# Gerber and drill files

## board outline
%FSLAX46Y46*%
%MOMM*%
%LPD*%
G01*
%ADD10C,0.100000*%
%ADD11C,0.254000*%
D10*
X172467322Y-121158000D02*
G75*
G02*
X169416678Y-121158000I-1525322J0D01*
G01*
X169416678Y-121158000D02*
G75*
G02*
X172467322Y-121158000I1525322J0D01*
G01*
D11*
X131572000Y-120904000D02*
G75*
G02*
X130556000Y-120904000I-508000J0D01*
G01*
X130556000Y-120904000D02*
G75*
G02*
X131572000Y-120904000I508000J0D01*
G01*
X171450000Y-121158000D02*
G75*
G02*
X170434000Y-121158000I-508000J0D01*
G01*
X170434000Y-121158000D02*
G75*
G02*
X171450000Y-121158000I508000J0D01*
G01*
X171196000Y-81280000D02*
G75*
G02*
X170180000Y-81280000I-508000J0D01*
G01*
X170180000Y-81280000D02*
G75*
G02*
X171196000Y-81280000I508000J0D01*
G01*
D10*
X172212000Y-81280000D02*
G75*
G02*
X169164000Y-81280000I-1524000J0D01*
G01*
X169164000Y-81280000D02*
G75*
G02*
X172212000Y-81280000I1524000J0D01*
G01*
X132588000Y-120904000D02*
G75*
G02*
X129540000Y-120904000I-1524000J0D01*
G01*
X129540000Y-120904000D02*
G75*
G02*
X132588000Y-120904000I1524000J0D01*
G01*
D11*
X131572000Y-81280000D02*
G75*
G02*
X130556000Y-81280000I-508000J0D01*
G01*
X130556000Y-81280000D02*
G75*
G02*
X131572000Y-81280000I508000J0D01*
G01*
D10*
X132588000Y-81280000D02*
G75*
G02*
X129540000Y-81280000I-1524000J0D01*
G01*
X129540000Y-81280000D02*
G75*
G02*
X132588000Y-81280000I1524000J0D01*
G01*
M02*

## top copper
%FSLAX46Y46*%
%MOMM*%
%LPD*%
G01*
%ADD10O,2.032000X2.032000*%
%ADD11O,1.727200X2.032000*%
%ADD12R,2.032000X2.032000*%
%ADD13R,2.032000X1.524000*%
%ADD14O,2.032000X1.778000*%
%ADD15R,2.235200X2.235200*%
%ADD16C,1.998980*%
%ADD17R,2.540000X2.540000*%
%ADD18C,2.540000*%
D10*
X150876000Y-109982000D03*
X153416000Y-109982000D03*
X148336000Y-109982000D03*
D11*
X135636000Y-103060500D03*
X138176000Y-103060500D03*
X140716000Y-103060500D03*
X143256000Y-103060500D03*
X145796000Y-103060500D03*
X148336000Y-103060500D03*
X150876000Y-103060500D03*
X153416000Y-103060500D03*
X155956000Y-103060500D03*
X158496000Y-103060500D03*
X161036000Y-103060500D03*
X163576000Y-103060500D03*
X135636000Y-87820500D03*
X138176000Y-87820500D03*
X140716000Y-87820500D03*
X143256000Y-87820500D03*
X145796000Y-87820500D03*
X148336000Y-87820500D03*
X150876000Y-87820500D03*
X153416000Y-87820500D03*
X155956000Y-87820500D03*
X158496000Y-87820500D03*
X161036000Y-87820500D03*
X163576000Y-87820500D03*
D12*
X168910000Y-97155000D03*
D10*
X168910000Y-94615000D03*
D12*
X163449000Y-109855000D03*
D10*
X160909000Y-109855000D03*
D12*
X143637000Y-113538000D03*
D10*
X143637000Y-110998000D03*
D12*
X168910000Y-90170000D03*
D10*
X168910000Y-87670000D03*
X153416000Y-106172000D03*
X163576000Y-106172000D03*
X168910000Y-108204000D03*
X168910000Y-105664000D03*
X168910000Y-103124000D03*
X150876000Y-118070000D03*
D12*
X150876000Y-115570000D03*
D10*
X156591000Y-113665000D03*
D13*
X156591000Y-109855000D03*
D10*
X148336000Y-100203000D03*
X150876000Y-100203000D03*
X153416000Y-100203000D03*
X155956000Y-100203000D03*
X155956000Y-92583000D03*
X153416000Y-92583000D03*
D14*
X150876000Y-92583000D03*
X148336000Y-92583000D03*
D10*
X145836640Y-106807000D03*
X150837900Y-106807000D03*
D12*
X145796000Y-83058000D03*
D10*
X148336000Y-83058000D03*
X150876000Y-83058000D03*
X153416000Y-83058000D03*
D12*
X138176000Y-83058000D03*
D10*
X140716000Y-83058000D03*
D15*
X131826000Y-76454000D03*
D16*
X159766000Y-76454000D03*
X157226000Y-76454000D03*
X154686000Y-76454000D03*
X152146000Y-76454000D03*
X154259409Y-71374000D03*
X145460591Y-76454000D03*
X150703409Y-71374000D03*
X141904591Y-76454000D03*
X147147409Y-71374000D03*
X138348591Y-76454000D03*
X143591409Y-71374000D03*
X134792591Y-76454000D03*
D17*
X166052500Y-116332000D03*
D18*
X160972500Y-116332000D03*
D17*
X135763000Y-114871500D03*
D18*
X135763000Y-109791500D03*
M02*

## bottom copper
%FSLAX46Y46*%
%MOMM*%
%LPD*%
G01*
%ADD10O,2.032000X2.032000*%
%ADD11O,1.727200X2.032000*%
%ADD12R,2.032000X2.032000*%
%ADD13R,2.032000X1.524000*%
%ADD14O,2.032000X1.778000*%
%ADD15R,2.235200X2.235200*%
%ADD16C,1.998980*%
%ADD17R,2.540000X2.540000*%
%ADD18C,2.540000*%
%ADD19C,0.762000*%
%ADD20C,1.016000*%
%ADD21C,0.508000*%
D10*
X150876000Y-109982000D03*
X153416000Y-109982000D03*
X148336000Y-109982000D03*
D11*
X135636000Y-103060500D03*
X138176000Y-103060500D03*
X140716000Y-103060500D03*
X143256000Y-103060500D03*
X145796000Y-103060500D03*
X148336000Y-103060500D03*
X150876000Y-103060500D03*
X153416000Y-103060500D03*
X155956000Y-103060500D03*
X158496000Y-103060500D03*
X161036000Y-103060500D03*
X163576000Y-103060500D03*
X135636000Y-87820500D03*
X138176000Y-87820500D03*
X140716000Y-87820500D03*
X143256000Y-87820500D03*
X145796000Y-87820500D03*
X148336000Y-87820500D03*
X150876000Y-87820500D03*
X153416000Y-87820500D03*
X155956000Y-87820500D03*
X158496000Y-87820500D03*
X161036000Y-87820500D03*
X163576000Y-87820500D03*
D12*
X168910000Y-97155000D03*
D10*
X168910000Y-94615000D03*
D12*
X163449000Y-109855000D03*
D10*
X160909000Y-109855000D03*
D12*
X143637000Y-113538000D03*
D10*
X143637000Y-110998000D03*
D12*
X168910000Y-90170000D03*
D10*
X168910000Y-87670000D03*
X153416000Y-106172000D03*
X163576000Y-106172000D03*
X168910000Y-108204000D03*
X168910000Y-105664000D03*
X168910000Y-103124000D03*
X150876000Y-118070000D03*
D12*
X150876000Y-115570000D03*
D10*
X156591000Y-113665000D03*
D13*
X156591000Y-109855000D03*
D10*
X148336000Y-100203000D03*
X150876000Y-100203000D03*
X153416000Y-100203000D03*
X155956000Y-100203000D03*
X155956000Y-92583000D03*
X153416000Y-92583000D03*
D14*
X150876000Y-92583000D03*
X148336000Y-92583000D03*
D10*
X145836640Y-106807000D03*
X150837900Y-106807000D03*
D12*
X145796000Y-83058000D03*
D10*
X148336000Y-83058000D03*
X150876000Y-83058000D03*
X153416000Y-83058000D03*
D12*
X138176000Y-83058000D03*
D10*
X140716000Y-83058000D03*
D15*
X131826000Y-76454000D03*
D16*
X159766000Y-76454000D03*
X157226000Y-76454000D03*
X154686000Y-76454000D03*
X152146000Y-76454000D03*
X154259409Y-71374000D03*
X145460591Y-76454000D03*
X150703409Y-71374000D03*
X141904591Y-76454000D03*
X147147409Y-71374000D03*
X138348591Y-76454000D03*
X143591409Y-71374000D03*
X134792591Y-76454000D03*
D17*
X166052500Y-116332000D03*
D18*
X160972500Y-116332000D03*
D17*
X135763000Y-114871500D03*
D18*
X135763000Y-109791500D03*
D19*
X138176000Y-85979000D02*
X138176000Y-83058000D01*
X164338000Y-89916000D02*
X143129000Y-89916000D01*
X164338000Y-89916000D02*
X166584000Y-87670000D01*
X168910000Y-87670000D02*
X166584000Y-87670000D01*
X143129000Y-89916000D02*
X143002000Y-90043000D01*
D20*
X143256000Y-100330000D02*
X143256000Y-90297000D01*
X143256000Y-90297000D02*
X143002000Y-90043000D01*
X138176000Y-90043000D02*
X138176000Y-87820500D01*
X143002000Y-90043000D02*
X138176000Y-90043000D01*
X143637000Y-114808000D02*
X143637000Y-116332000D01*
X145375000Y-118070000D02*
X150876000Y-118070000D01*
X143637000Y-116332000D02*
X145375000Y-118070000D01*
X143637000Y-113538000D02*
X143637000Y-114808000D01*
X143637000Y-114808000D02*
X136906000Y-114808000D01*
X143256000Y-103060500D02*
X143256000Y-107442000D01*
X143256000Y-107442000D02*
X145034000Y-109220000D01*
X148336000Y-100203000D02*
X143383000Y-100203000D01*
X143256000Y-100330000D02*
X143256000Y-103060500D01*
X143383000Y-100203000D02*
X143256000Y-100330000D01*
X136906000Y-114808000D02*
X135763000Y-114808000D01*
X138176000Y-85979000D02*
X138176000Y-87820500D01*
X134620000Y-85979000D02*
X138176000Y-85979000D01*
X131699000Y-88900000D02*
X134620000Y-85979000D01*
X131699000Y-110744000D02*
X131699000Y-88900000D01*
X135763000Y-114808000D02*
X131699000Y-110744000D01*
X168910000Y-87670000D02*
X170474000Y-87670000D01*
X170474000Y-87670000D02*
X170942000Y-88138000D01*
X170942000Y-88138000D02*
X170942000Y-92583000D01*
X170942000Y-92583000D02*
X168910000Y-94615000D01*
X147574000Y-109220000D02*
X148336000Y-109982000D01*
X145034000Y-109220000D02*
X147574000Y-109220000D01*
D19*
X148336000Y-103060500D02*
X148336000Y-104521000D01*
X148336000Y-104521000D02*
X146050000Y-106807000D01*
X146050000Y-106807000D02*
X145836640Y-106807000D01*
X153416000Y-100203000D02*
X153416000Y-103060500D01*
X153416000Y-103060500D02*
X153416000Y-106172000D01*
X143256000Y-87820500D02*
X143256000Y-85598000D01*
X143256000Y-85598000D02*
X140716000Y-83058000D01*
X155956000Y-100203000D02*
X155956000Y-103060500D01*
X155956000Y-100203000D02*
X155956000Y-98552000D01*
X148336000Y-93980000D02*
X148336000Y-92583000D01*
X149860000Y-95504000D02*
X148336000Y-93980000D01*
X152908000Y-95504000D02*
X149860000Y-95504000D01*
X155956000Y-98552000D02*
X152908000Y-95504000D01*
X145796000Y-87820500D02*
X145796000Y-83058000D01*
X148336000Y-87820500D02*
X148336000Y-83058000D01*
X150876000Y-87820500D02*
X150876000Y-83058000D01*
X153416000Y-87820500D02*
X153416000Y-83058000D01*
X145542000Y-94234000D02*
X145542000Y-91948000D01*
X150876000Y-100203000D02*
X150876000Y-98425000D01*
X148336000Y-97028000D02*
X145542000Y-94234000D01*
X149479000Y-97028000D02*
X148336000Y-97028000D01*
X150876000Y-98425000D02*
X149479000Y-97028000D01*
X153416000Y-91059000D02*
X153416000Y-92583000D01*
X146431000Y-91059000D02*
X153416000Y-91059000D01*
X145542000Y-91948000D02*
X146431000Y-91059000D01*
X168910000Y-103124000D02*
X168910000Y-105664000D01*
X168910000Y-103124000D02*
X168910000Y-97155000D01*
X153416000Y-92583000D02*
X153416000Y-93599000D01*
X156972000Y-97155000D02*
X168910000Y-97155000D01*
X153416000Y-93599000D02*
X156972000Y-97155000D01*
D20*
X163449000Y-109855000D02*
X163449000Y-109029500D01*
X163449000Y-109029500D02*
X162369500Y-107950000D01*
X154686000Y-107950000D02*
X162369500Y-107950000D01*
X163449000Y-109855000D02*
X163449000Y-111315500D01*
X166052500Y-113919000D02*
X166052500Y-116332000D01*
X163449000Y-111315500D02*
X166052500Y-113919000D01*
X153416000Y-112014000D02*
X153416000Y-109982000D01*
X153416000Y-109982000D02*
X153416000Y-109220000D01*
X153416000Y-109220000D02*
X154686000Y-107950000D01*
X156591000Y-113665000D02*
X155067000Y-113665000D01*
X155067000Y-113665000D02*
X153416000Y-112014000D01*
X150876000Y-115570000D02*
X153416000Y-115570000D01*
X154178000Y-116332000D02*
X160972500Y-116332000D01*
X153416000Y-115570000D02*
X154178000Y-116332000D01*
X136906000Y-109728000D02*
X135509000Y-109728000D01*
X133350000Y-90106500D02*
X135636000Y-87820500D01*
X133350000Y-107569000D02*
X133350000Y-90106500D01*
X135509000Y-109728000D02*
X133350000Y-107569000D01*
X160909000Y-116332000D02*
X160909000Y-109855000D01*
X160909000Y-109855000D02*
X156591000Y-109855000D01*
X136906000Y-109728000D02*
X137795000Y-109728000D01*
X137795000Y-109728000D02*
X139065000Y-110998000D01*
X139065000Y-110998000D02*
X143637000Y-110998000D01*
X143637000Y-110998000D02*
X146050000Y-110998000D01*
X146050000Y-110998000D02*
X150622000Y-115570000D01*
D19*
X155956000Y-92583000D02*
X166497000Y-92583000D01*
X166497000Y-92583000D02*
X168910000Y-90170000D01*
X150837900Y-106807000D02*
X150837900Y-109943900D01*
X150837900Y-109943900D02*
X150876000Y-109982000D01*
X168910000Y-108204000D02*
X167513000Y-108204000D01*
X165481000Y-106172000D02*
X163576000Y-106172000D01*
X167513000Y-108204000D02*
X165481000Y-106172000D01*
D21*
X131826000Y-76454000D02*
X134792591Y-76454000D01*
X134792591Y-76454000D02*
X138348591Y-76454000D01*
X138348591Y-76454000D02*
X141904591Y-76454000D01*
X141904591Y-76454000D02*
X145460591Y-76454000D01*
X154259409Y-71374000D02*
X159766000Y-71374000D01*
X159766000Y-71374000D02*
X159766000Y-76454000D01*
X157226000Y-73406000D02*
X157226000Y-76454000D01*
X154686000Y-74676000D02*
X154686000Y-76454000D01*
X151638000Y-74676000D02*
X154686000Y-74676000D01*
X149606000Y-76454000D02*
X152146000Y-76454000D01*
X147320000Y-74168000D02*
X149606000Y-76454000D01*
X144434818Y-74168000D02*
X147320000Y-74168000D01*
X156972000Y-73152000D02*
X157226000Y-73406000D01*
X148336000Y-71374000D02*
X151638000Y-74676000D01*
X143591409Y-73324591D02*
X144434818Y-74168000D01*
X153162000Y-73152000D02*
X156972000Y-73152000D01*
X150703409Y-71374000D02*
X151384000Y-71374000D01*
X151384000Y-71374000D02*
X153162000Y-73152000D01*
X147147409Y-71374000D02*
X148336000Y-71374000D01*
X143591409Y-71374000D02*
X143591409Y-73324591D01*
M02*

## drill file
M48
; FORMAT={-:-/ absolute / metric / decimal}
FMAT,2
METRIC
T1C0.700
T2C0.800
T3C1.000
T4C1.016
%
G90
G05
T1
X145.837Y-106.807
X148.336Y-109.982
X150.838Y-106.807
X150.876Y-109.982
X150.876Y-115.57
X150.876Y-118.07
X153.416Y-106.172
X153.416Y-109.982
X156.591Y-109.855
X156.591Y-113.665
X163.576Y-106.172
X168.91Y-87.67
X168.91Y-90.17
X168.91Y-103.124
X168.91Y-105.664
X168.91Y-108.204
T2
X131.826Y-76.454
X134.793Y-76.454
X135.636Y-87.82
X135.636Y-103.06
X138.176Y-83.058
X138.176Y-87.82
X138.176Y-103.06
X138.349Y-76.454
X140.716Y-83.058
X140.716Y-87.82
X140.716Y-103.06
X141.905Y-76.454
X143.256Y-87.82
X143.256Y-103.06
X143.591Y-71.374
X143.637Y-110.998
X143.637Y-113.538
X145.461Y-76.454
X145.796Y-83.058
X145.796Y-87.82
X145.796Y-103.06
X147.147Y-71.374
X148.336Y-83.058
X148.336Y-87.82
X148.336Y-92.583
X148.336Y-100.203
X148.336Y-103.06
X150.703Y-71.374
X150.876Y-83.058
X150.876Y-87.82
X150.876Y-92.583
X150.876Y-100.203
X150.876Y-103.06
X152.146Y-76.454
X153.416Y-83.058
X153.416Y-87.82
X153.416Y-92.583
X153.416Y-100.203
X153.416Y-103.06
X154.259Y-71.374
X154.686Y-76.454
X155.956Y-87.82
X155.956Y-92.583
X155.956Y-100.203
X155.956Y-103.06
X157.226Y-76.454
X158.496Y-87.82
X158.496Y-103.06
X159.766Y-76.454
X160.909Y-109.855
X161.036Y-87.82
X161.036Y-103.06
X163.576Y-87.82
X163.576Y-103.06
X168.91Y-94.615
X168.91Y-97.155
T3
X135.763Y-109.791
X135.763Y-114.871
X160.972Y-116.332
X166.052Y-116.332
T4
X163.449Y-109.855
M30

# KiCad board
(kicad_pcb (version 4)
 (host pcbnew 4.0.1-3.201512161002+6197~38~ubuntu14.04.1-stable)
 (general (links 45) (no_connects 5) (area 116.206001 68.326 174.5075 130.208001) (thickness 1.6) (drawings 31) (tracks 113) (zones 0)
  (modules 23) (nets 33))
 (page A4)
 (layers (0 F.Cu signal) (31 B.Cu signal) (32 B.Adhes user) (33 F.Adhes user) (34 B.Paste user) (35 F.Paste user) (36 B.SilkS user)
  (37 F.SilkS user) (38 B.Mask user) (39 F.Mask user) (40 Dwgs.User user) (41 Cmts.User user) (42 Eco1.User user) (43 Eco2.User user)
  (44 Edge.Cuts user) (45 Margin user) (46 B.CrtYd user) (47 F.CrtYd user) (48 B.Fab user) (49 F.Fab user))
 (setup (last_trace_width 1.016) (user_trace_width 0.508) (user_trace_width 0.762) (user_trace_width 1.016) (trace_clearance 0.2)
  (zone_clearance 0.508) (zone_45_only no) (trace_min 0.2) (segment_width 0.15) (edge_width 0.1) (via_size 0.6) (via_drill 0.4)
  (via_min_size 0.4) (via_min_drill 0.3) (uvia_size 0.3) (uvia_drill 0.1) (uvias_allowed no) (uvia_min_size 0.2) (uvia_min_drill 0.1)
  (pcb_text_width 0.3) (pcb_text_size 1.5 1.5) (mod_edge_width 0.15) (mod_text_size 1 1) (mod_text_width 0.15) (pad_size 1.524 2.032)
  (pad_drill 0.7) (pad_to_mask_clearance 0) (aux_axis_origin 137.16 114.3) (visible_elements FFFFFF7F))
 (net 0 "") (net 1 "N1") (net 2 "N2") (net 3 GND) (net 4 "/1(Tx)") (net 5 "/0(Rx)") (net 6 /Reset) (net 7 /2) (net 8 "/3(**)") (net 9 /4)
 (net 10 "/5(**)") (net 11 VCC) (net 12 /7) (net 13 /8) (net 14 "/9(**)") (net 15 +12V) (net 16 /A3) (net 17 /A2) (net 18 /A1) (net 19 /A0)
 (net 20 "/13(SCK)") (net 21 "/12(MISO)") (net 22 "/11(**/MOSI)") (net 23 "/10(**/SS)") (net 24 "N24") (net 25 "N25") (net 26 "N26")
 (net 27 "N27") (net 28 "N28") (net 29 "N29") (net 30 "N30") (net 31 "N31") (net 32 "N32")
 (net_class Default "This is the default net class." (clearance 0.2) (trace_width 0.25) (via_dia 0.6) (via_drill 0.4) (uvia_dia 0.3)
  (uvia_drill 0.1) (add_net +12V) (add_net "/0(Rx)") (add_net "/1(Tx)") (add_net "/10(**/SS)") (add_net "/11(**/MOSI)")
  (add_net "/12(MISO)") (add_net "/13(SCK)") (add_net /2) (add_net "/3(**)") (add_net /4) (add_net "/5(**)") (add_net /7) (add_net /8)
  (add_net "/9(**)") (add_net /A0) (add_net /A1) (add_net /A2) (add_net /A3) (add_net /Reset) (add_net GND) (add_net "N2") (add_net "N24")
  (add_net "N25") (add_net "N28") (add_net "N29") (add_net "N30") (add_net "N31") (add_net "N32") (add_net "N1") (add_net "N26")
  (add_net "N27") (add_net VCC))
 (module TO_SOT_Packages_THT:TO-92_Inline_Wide (layer F.Cu) (at 148.336 109.982)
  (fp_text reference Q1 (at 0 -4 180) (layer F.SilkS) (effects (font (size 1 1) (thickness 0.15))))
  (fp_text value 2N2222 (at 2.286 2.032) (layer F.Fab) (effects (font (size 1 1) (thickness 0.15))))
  (pad 2 thru_hole oval (at 2.54 0) (size 2.032 2.032) (drill 0.7) (layers *.Cu *.Mask F.SilkS) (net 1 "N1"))
  (pad 3 thru_hole oval (at 5.08 0) (size 2.032 2.032) (drill 0.7) (layers *.Cu *.Mask F.SilkS) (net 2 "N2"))
  (pad 1 thru_hole oval (at 0 0) (size 2.032 2.032) (drill 0.7) (layers *.Cu *.Mask F.SilkS) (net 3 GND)))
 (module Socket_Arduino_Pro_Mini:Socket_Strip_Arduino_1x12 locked (layer F.Cu) (at 135.636 103.0605)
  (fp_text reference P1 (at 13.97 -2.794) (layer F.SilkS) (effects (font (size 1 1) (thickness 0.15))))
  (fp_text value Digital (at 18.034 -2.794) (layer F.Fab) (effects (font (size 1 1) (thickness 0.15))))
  (pad 1 thru_hole oval (at 0 0) (size 1.7272 2.032) (drill 0.8) (layers *.Cu *.Mask F.SilkS) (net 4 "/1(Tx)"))
  (pad 2 thru_hole oval (at 2.54 0) (size 1.7272 2.032) (drill 0.8) (layers *.Cu *.Mask F.SilkS) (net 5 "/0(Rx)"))
  (pad 3 thru_hole oval (at 5.08 0) (size 1.7272 2.032) (drill 0.8) (layers *.Cu *.Mask F.SilkS) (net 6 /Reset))
  (pad 4 thru_hole oval (at 7.62 0) (size 1.7272 2.032) (drill 0.8) (layers *.Cu *.Mask F.SilkS) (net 3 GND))
  (pad 5 thru_hole oval (at 10.16 0) (size 1.7272 2.032) (drill 0.8) (layers *.Cu *.Mask F.SilkS) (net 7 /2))
  (pad 6 thru_hole oval (at 12.7 0) (size 1.7272 2.032) (drill 0.8) (layers *.Cu *.Mask F.SilkS) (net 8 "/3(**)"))
  (pad 7 thru_hole oval (at 15.24 0) (size 1.7272 2.032) (drill 0.8) (layers *.Cu *.Mask F.SilkS) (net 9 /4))
  (pad 8 thru_hole oval (at 17.78 0) (size 1.7272 2.032) (drill 0.8) (layers *.Cu *.Mask F.SilkS) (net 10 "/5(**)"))
  (pad 9 thru_hole oval (at 20.32 0) (size 1.7272 2.032) (drill 0.8) (layers *.Cu *.Mask F.SilkS) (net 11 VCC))
  (pad 10 thru_hole oval (at 22.86 0) (size 1.7272 2.032) (drill 0.8) (layers *.Cu *.Mask F.SilkS) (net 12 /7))
  (pad 11 thru_hole oval (at 25.4 0) (size 1.7272 2.032) (drill 0.8) (layers *.Cu *.Mask F.SilkS) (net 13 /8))
  (pad 12 thru_hole oval (at 27.94 0) (size 1.7272 2.032) (drill 0.8) (layers *.Cu *.Mask F.SilkS) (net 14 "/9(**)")))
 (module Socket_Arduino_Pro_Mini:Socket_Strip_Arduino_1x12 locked (layer F.Cu) (at 135.636 87.8205)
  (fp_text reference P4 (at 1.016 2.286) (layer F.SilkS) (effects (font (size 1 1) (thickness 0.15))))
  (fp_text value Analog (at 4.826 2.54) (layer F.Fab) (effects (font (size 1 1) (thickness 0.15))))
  (pad 1 thru_hole oval (at 0 0) (size 1.7272 2.032) (drill 0.8) (layers *.Cu *.Mask F.SilkS) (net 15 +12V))
  (pad 2 thru_hole oval (at 2.54 0) (size 1.7272 2.032) (drill 0.8) (layers *.Cu *.Mask F.SilkS) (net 3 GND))
  (pad 3 thru_hole oval (at 5.08 0) (size 1.7272 2.032) (drill 0.8) (layers *.Cu *.Mask F.SilkS) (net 6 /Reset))
  (pad 4 thru_hole oval (at 7.62 0) (size 1.7272 2.032) (drill 0.8) (layers *.Cu *.Mask F.SilkS) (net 11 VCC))
  (pad 5 thru_hole oval (at 10.16 0) (size 1.7272 2.032) (drill 0.8) (layers *.Cu *.Mask F.SilkS) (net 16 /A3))
  (pad 6 thru_hole oval (at 12.7 0) (size 1.7272 2.032) (drill 0.8) (layers *.Cu *.Mask F.SilkS) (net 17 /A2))
  (pad 7 thru_hole oval (at 15.24 0) (size 1.7272 2.032) (drill 0.8) (layers *.Cu *.Mask F.SilkS) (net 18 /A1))
  (pad 8 thru_hole oval (at 17.78 0) (size 1.7272 2.032) (drill 0.8) (layers *.Cu *.Mask F.SilkS) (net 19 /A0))
  (pad 9 thru_hole oval (at 20.32 0) (size 1.7272 2.032) (drill 0.8) (layers *.Cu *.Mask F.SilkS) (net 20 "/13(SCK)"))
  (pad 10 thru_hole oval (at 22.86 0) (size 1.7272 2.032) (drill 0.8) (layers *.Cu *.Mask F.SilkS) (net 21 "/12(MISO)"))
  (pad 11 thru_hole oval (at 25.4 0) (size 1.7272 2.032) (drill 0.8) (layers *.Cu *.Mask F.SilkS) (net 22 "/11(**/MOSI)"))
  (pad 12 thru_hole oval (at 27.94 0) (size 1.7272 2.032) (drill 0.8) (layers *.Cu *.Mask F.SilkS) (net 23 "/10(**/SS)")))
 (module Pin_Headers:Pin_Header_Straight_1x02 (layer F.Cu) (at 168.91 97.155 180)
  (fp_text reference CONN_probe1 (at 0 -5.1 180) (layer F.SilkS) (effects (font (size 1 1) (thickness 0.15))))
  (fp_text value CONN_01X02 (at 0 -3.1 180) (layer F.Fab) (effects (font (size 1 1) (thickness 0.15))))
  (pad 1 thru_hole rect (at 0 0 180) (size 2.032 2.032) (drill 0.8) (layers *.Cu *.Mask F.SilkS) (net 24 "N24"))
  (pad 2 thru_hole oval (at 0 2.54 180) (size 2.032 2.032) (drill 0.8) (layers *.Cu *.Mask F.SilkS) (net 3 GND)))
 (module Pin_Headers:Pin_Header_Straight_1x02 (layer F.Cu) (at 163.449 109.855 270)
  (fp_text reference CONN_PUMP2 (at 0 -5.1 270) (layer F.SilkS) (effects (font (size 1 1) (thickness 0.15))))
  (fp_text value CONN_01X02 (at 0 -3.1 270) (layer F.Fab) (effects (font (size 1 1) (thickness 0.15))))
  (pad 1 thru_hole rect (at 0 0 270) (size 2.032 2.032) (drill 1.016) (layers *.Cu *.Mask F.SilkS) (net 2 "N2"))
  (pad 2 thru_hole oval (at 0 2.54 270) (size 2.032 2.032) (drill 0.8) (layers *.Cu *.Mask F.SilkS) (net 15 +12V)))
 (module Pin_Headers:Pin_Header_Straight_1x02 (layer F.Cu) (at 143.637 113.538 180)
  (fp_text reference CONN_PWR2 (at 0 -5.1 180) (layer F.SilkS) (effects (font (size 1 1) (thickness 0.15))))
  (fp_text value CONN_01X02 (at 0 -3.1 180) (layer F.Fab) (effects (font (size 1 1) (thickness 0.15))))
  (pad 1 thru_hole rect (at 0 0 180) (size 2.032 2.032) (drill 0.8) (layers *.Cu *.Mask F.SilkS) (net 3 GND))
  (pad 2 thru_hole oval (at 0 2.54 180) (size 2.032 2.032) (drill 0.8) (layers *.Cu *.Mask F.SilkS) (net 15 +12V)))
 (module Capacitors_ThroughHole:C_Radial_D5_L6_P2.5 (layer F.Cu) (at 168.91 90.17 90)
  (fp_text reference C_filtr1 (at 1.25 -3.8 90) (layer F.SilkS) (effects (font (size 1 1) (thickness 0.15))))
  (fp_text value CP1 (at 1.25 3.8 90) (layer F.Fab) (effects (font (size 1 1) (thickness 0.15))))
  (pad 1 thru_hole rect (at 0 0 90) (size 2.032 2.032) (drill 0.7) (layers *.Cu *.Mask F.SilkS) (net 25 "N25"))
  (pad 2 thru_hole oval (at 2.5 0 90) (size 2.032 2.032) (drill 0.7) (layers *.Cu *.Mask F.SilkS) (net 3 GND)))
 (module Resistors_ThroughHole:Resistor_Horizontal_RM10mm (layer F.Cu) (at 158.496 106.172)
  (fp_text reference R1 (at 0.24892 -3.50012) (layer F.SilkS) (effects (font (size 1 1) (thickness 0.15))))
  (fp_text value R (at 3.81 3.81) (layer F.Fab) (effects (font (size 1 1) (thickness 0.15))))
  (pad 1 thru_hole oval (at -5.08 0) (size 2.032 2.032) (drill 0.7) (layers *.Cu *.Mask F.SilkS) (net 10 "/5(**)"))
  (pad 2 thru_hole oval (at 5.08 0) (size 2.032 2.032) (drill 0.7) (layers *.Cu *.Mask F.SilkS) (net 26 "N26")))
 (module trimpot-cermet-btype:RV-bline (layer F.Cu) (at 168.91 105.664 90)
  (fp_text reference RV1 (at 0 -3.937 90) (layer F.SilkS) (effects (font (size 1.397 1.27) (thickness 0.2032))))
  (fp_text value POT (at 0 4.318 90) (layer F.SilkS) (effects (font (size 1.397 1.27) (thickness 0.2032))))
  (pad 1 thru_hole oval (at -2.54 0 90) (size 2.032 2.032) (drill 0.7) (layers *.Cu *.Mask F.SilkS) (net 26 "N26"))
  (pad 2 thru_hole oval (at 0 0 90) (size 2.032 2.032) (drill 0.7) (layers *.Cu *.Mask F.SilkS) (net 24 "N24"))
  (pad 3 thru_hole oval (at 2.54 0 90) (size 2.032 2.032) (drill 0.7) (layers *.Cu *.Mask F.SilkS) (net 24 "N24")))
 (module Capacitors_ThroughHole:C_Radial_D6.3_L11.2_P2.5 (layer F.Cu) (at 150.876 115.57 270)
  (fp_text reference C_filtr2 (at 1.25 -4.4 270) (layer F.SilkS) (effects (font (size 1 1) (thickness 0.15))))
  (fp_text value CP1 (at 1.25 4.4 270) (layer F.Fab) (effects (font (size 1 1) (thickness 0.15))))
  (pad 2 thru_hole oval (at 2.5 0 270) (size 2.032 2.032) (drill 0.7) (layers *.Cu *.Mask F.SilkS) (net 3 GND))
  (pad 1 thru_hole rect (at 0 0 270) (size 2.032 2.032) (drill 0.7) (layers *.Cu *.Mask F.SilkS) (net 15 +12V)))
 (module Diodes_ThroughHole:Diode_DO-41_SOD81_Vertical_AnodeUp (layer F.Cu) (at 156.591 109.855 270)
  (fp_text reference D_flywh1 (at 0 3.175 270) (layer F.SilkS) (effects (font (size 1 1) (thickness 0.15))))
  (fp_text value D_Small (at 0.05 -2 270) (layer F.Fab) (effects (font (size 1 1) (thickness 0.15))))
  (pad 2 thru_hole oval (at 3.81 0 270) (size 2.032 2.032) (drill 0.7) (layers *.Cu *.Mask F.SilkS) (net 2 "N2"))
  (pad 1 thru_hole rect (at 0 0 270) (size 1.524 2.032) (drill 0.7) (layers *.Cu *.Mask F.SilkS) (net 15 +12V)))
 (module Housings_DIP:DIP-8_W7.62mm (layer F.Cu) (at 148.336 100.203 90)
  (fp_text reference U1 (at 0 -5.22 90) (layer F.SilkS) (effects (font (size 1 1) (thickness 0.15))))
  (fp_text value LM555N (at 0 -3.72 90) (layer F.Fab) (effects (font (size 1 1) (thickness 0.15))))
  (pad 1 thru_hole oval (at 0 0 90) (size 2.032 2.032) (drill 0.8) (layers *.Cu *.Mask F.SilkS) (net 3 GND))
  (pad 2 thru_hole oval (at 0 2.54 90) (size 2.032 2.032) (drill 0.8) (layers *.Cu *.Mask F.SilkS) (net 24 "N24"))
  (pad 3 thru_hole oval (at 0 5.08 90) (size 2.032 2.032) (drill 0.8) (layers *.Cu *.Mask F.SilkS) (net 10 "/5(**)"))
  (pad 4 thru_hole oval (at 0 7.62 90) (size 2.032 2.032) (drill 0.8) (layers *.Cu *.Mask F.SilkS) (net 11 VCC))
  (pad 5 thru_hole oval (at 7.62 7.62 90) (size 2.032 2.032) (drill 0.8) (layers *.Cu *.Mask F.SilkS) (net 25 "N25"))
  (pad 6 thru_hole oval (at 7.62 5.08 90) (size 2.032 2.032) (drill 0.8) (layers *.Cu *.Mask F.SilkS) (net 24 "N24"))
  (pad 7 thru_hole oval (at 7.62 2.54 90) (size 1.778 2.032) (drill 0.8) (layers *.Cu *.Mask F.SilkS) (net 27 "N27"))
  (pad 8 thru_hole oval (at 7.62 0 90) (size 1.778 2.032) (drill 0.8) (layers *.Cu *.Mask F.SilkS) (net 11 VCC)))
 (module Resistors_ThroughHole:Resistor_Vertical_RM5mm (layer F.Cu) (at 148.336 106.807)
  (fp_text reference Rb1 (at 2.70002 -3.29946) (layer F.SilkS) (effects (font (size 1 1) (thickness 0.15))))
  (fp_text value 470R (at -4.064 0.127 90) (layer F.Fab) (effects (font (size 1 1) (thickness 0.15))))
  (pad 1 thru_hole oval (at -2.49936 0) (size 2.032 2.032) (drill 0.7) (layers *.Cu *.Mask F.SilkS) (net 8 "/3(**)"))
  (pad 2 thru_hole oval (at 2.5019 0) (size 2.032 2.032) (drill 0.7) (layers *.Cu *.Mask F.SilkS) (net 1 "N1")))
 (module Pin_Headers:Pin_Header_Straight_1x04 (layer F.Cu) (at 145.796 83.058 90)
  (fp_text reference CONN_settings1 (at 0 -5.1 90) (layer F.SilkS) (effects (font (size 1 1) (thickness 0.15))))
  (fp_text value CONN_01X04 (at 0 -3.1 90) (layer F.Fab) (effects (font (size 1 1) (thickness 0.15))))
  (pad 1 thru_hole rect (at 0 0 90) (size 2.032 2.032) (drill 0.8) (layers *.Cu *.Mask F.SilkS) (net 16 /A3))
  (pad 2 thru_hole oval (at 0 2.54 90) (size 2.032 2.032) (drill 0.8) (layers *.Cu *.Mask F.SilkS) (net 17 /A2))
  (pad 3 thru_hole oval (at 0 5.08 90) (size 2.032 2.032) (drill 0.8) (layers *.Cu *.Mask F.SilkS) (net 18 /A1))
  (pad 4 thru_hole oval (at 0 7.62 90) (size 2.032 2.032) (drill 0.8) (layers *.Cu *.Mask F.SilkS) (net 19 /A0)))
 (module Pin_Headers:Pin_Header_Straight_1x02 (layer F.Cu) (at 138.176 83.058 90)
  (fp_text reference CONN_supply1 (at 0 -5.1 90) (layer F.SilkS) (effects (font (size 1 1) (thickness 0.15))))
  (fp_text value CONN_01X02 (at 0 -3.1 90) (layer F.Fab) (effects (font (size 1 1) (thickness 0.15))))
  (pad 1 thru_hole rect (at 0 0 90) (size 2.032 2.032) (drill 0.8) (layers *.Cu *.Mask F.SilkS) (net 3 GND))
  (pad 2 thru_hole oval (at 0 2.54 90) (size 2.032 2.032) (drill 0.8) (layers *.Cu *.Mask F.SilkS) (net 11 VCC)))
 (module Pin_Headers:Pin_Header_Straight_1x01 (layer F.Cu) (at 131.826 76.454)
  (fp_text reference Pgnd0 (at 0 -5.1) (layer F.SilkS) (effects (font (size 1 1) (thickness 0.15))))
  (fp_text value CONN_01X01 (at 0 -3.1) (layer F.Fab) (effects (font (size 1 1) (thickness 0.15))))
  (pad 1 thru_hole rect (at 0 0) (size 2.2352 2.2352) (drill 0.8) (layers *.Cu *.Mask F.SilkS) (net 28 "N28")))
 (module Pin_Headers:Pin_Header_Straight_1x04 (layer F.Cu) (at 159.766 76.454 270)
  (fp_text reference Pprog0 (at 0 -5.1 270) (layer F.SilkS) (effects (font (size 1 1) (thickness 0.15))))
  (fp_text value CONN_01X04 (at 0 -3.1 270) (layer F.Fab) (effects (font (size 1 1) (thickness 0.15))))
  (pad 1 thru_hole circle (at 0 0 270) (size 1.99898 1.99898) (drill 0.8) (layers *.Cu *.SilkS *.Mask) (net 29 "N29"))
  (pad 2 thru_hole circle (at 0 2.54 270) (size 1.99898 1.99898) (drill 0.8) (layers *.Cu *.SilkS *.Mask) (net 29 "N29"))
  (pad 3 thru_hole circle (at 0 5.08 270) (size 1.99898 1.99898) (drill 0.8) (layers *.Cu *.SilkS *.Mask) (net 29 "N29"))
  (pad 4 thru_hole circle (at 0 7.62 270) (size 1.99898 1.99898) (drill 0.8) (layers *.Cu *.SilkS *.Mask) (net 29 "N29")))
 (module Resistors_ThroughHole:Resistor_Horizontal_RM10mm (layer F.Cu) (at 149.86 73.914 210)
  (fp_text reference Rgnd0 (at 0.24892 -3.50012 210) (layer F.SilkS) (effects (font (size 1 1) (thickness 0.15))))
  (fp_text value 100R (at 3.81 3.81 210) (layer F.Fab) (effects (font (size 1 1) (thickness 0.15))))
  (pad 1 thru_hole circle (at -5.08 0 210) (size 1.99898 1.99898) (drill 0.8) (layers *.Cu *.SilkS *.Mask) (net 29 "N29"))
  (pad 2 thru_hole circle (at 5.08 0 210) (size 1.99898 1.99898) (drill 0.8) (layers *.Cu *.SilkS *.Mask) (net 28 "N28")))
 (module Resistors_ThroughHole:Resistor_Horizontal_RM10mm (layer F.Cu) (at 146.304 73.914 210)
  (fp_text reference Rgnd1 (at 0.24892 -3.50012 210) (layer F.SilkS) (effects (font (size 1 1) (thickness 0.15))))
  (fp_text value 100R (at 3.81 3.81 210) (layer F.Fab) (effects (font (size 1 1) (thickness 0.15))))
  (pad 1 thru_hole circle (at -5.08 0 210) (size 1.99898 1.99898) (drill 0.8) (layers *.Cu *.SilkS *.Mask) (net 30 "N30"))
  (pad 2 thru_hole circle (at 5.08 0 210) (size 1.99898 1.99898) (drill 0.8) (layers *.Cu *.SilkS *.Mask) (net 28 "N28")))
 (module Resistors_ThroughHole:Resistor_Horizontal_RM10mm (layer F.Cu) (at 142.748 73.914 210)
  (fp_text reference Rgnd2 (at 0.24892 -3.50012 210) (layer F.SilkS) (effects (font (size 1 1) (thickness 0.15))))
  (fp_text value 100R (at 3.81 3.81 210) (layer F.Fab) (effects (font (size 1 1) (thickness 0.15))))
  (pad 1 thru_hole circle (at -5.08 0 210) (size 1.99898 1.99898) (drill 0.8) (layers *.Cu *.SilkS *.Mask) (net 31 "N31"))
  (pad 2 thru_hole circle (at 5.08 0 210) (size 1.99898 1.99898) (drill 0.8) (layers *.Cu *.SilkS *.Mask) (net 28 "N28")))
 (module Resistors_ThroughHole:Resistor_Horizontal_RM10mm (layer F.Cu) (at 139.192 73.914 210)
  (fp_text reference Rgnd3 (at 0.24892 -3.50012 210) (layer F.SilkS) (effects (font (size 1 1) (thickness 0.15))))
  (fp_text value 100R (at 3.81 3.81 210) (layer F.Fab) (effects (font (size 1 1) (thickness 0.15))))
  (pad 1 thru_hole circle (at -5.08 0 210) (size 1.99898 1.99898) (drill 0.8) (layers *.Cu *.SilkS *.Mask) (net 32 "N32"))
  (pad 2 thru_hole circle (at 5.08 0 210) (size 1.99898 1.99898) (drill 0.8) (layers *.Cu *.SilkS *.Mask) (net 28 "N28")))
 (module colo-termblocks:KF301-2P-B (layer F.Cu) (at 163.5125 116.332)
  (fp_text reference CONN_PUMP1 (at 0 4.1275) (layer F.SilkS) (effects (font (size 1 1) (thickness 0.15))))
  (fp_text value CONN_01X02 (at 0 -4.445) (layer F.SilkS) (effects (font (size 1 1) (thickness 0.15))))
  (pad 1 thru_hole rect (at 2.54 0) (size 2.54 2.54) (drill 1) (layers *.Cu *.Mask F.SilkS) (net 2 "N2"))
  (pad 2 thru_hole circle (at -2.54 0) (size 2.54 2.54) (drill 1) (layers *.Cu *.Mask F.SilkS) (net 15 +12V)))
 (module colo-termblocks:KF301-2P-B (layer F.Cu) (at 135.763 112.3315 270)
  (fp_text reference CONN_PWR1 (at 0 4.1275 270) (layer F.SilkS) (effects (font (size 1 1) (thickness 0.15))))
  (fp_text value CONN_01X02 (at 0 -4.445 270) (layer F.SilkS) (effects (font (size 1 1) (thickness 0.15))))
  (pad 1 thru_hole rect (at 2.54 0 270) (size 2.54 2.54) (drill 1) (layers *.Cu *.Mask F.SilkS) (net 3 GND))
  (pad 2 thru_hole circle (at -2.54 0 270) (size 2.54 2.54) (drill 1) (layers *.Cu *.Mask F.SilkS) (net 15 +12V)))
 (gr_circle (center 170.942 121.158) (end 172.466 121.2215) (layer Edge.Cuts) (width 0.1))
 (gr_circle (center 131.064 120.904) (end 130.556 120.904) (layer Edge.Cuts) (width 0.254))
 (gr_circle (center 170.942 121.158) (end 170.434 121.158) (layer Edge.Cuts) (width 0.254))
 (gr_circle (center 170.688 81.28) (end 170.18 81.28) (layer Edge.Cuts) (width 0.254))
 (gr_circle (center 170.688 81.28) (end 169.164 81.28) (layer Edge.Cuts) (width 0.1))
 (gr_circle (center 131.064 120.904) (end 129.54 120.904) (layer Edge.Cuts) (width 0.1))
 (gr_circle (center 131.064 81.28) (end 130.556 81.28) (layer Edge.Cuts) (width 0.254))
 (gr_circle (center 131.064 81.28) (end 129.54 81.28) (layer Edge.Cuts) (width 0.1))
 (segment (start 138.176 85.979) (end 138.176 83.058) (width 0.762) (layer B.Cu) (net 3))
 (segment (start 164.338 89.916) (end 143.129 89.916) (width 0.762) (layer B.Cu) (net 3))
 (segment (start 164.338 89.916) (end 166.584 87.67) (width 0.762) (layer B.Cu) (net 3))
 (segment (start 168.91 87.67) (end 166.584 87.67) (width 0.762) (layer B.Cu) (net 3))
 (segment (start 143.129 89.916) (end 143.002 90.043) (width 0.762) (layer B.Cu) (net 3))
 (segment (start 143.256 100.33) (end 143.256 90.297) (width 1.016) (layer B.Cu) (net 3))
 (segment (start 143.256 90.297) (end 143.002 90.043) (width 1.016) (layer B.Cu) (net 3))
 (segment (start 138.176 90.043) (end 138.176 87.8205) (width 1.016) (layer B.Cu) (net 3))
 (segment (start 143.002 90.043) (end 138.176 90.043) (width 1.016) (layer B.Cu) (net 3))
 (segment (start 143.637 114.808) (end 143.637 116.332) (width 1.016) (layer B.Cu) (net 3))
 (segment (start 145.375 118.07) (end 150.876 118.07) (width 1.016) (layer B.Cu) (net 3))
 (segment (start 143.637 116.332) (end 145.375 118.07) (width 1.016) (layer B.Cu) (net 3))
 (segment (start 143.637 113.538) (end 143.637 114.808) (width 1.016) (layer B.Cu) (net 3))
 (segment (start 143.637 114.808) (end 136.906 114.808) (width 1.016) (layer B.Cu) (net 3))
 (segment (start 143.256 103.0605) (end 143.256 107.442) (width 1.016) (layer B.Cu) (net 3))
 (segment (start 143.256 107.442) (end 145.034 109.22) (width 1.016) (layer B.Cu) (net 3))
 (segment (start 148.336 100.203) (end 143.383 100.203) (width 1.016) (layer B.Cu) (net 3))
 (segment (start 143.256 100.33) (end 143.256 103.0605) (width 1.016) (layer B.Cu) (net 3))
 (segment (start 143.383 100.203) (end 143.256 100.33) (width 1.016) (layer B.Cu) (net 3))
 (segment (start 136.906 114.808) (end 135.763 114.808) (width 1.016) (layer B.Cu) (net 3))
 (segment (start 138.176 85.979) (end 138.176 87.8205) (width 1.016) (layer B.Cu) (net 3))
 (segment (start 134.62 85.979) (end 138.176 85.979) (width 1.016) (layer B.Cu) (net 3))
 (segment (start 131.699 88.9) (end 134.62 85.979) (width 1.016) (layer B.Cu) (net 3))
 (segment (start 131.699 110.744) (end 131.699 88.9) (width 1.016) (layer B.Cu) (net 3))
 (segment (start 135.763 114.808) (end 131.699 110.744) (width 1.016) (layer B.Cu) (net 3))
 (segment (start 168.91 87.67) (end 170.474 87.67) (width 1.016) (layer B.Cu) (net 3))
 (segment (start 170.474 87.67) (end 170.942 88.138) (width 1.016) (layer B.Cu) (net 3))
 (segment (start 170.942 88.138) (end 170.942 92.583) (width 1.016) (layer B.Cu) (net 3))
 (segment (start 170.942 92.583) (end 168.91 94.615) (width 1.016) (layer B.Cu) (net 3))
 (segment (start 147.574 109.22) (end 148.336 109.982) (width 1.016) (layer B.Cu) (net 3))
 (segment (start 145.034 109.22) (end 147.574 109.22) (width 1.016) (layer B.Cu) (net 3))
 (segment (start 148.336 103.0605) (end 148.336 104.521) (width 0.762) (layer B.Cu) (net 8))
 (segment (start 148.336 104.521) (end 146.05 106.807) (width 0.762) (layer B.Cu) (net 8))
 (segment (start 146.05 106.807) (end 145.83664 106.807) (width 0.762) (layer B.Cu) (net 8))
 (segment (start 153.416 100.203) (end 153.416 103.0605) (width 0.762) (layer B.Cu) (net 10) (status 10))
 (segment (start 153.416 103.0605) (end 153.416 106.172) (width 0.762) (layer B.Cu) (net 10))
 (segment (start 143.256 87.8205) (end 143.256 85.598) (width 0.762) (layer B.Cu) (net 11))
 (segment (start 143.256 85.598) (end 140.716 83.058) (width 0.762) (layer B.Cu) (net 11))
 (segment (start 155.956 100.203) (end 155.956 103.0605) (width 0.762) (layer B.Cu) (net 11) (status 10))
 (segment (start 155.956 100.203) (end 155.956 98.552) (width 0.762) (layer B.Cu) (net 11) (status 10))
 (segment (start 148.336 93.98) (end 148.336 92.583) (width 0.762) (layer B.Cu) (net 11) (status 20))
 (segment (start 149.86 95.504) (end 148.336 93.98) (width 0.762) (layer B.Cu) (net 11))
 (segment (start 152.908 95.504) (end 149.86 95.504) (width 0.762) (layer B.Cu) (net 11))
 (segment (start 155.956 98.552) (end 152.908 95.504) (width 0.762) (layer B.Cu) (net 11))
 (segment (start 145.796 87.8205) (end 145.796 83.058) (width 0.762) (layer B.Cu) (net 16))
 (segment (start 148.336 87.8205) (end 148.336 83.058) (width 0.762) (layer B.Cu) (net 17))
 (segment (start 150.876 87.8205) (end 150.876 83.058) (width 0.762) (layer B.Cu) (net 18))
 (segment (start 153.416 87.8205) (end 153.416 83.058) (width 0.762) (layer B.Cu) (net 19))
 (segment (start 145.542 94.234) (end 145.542 91.948) (width 0.762) (layer B.Cu) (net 24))
 (segment (start 150.876 100.203) (end 150.876 98.425) (width 0.762) (layer B.Cu) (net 24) (status 10))
 (segment (start 148.336 97.028) (end 145.542 94.234) (width 0.762) (layer B.Cu) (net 24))
 (segment (start 149.479 97.028) (end 148.336 97.028) (width 0.762) (layer B.Cu) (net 24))
 (segment (start 150.876 98.425) (end 149.479 97.028) (width 0.762) (layer B.Cu) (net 24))
 (segment (start 153.416 91.059) (end 153.416 92.583) (width 0.762) (layer B.Cu) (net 24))
 (segment (start 146.431 91.059) (end 153.416 91.059) (width 0.762) (layer B.Cu) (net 24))
 (segment (start 145.542 91.948) (end 146.431 91.059) (width 0.762) (layer B.Cu) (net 24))
 (segment (start 168.91 103.124) (end 168.91 105.664) (width 0.762) (layer B.Cu) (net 24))
 (segment (start 168.91 103.124) (end 168.91 97.155) (width 0.762) (layer B.Cu) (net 24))
 (segment (start 153.416 92.583) (end 153.416 93.599) (width 0.762) (layer B.Cu) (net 24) (status 10))
 (segment (start 156.972 97.155) (end 168.91 97.155) (width 0.762) (layer B.Cu) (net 24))
 (segment (start 153.416 93.599) (end 156.972 97.155) (width 0.762) (layer B.Cu) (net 24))
 (segment (start 163.449 109.855) (end 163.449 109.0295) (width 1.016) (layer B.Cu) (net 2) (status C00000))
 (segment (start 163.449 109.0295) (end 162.3695 107.95) (width 1.016) (layer B.Cu) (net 2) (status 400000))
 (segment (start 154.686 107.95) (end 162.3695 107.95) (width 1.016) (layer B.Cu) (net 2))
 (segment (start 163.449 109.855) (end 163.449 111.3155) (width 1.016) (layer B.Cu) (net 2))
 (segment (start 166.0525 113.919) (end 166.0525 116.332) (width 1.016) (layer B.Cu) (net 2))
 (segment (start 163.449 111.3155) (end 166.0525 113.919) (width 1.016) (layer B.Cu) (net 2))
 (segment (start 153.416 112.014) (end 153.416 109.982) (width 1.016) (layer B.Cu) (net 2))
 (segment (start 153.416 109.982) (end 153.416 109.22) (width 1.016) (layer B.Cu) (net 2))
 (segment (start 153.416 109.22) (end 154.686 107.95) (width 1.016) (layer B.Cu) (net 2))
 (segment (start 156.591 113.665) (end 155.067 113.665) (width 1.016) (layer B.Cu) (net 2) (status 10))
 (segment (start 155.067 113.665) (end 153.416 112.014) (width 1.016) (layer B.Cu) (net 2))
 (segment (start 150.876 115.57) (end 153.416 115.57) (width 1.016) (layer B.Cu) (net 15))
 (segment (start 154.178 116.332) (end 160.9725 116.332) (width 1.016) (layer B.Cu) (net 15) (status 20))
 (segment (start 153.416 115.57) (end 154.178 116.332) (width 1.016) (layer B.Cu) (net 15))
 (segment (start 136.906 109.728) (end 135.509 109.728) (width 1.016) (layer B.Cu) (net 15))
 (segment (start 133.35 90.1065) (end 135.636 87.8205) (width 1.016) (layer B.Cu) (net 15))
 (segment (start 133.35 107.569) (end 133.35 90.1065) (width 1.016) (layer B.Cu) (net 15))
 (segment (start 135.509 109.728) (end 133.35 107.569) (width 1.016) (layer B.Cu) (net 15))
 (segment (start 160.909 116.332) (end 160.909 109.855) (width 1.016) (layer B.Cu) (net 15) (status 10))
 (segment (start 160.909 109.855) (end 156.591 109.855) (width 1.016) (layer B.Cu) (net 15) (status 10))
 (segment (start 136.906 109.728) (end 137.795 109.728) (width 1.016) (layer B.Cu) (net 15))
 (segment (start 137.795 109.728) (end 139.065 110.998) (width 1.016) (layer B.Cu) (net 15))
 (segment (start 139.065 110.998) (end 143.637 110.998) (width 1.016) (layer B.Cu) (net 15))
 (segment (start 143.637 110.998) (end 146.05 110.998) (width 1.016) (layer B.Cu) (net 15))
 (segment (start 146.05 110.998) (end 150.622 115.57) (width 1.016) (layer B.Cu) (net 15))
 (segment (start 155.956 92.583) (end 166.497 92.583) (width 0.762) (layer B.Cu) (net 25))
 (segment (start 166.497 92.583) (end 168.91 90.17) (width 0.762) (layer B.Cu) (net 25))
 (segment (start 150.8379 106.807) (end 150.8379 109.9439) (width 0.762) (layer B.Cu) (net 1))
 (segment (start 150.8379 109.9439) (end 150.876 109.982) (width 0.762) (layer B.Cu) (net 1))
 (segment (start 168.91 108.204) (end 167.513 108.204) (width 0.762) (layer B.Cu) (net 26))
 (segment (start 165.481 106.172) (end 163.576 106.172) (width 0.762) (layer B.Cu) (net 26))
 (segment (start 167.513 108.204) (end 165.481 106.172) (width 0.762) (layer B.Cu) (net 26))
 (segment (start 131.826 76.454) (end 134.792591 76.454) (width 0.508) (layer B.Cu) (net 28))
 (segment (start 134.792591 76.454) (end 138.348591 76.454) (width 0.508) (layer B.Cu) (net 28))
 (segment (start 138.348591 76.454) (end 141.904591 76.454) (width 0.508) (layer B.Cu) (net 28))
 (segment (start 141.904591 76.454) (end 145.460591 76.454) (width 0.508) (layer B.Cu) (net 28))
 (segment (start 154.259409 71.374) (end 159.766 71.374) (width 0.508) (layer B.Cu) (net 29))
 (segment (start 159.766 71.374) (end 159.766 76.454) (width 0.508) (layer B.Cu) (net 29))
 (segment (start 157.226 73.406) (end 157.226 76.454) (width 0.508) (layer B.Cu) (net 29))
 (segment (start 154.686 74.676) (end 154.686 76.454) (width 0.508) (layer B.Cu) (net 29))
 (segment (start 151.638 74.676) (end 154.686 74.676) (width 0.508) (layer B.Cu) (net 29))
 (segment (start 149.606 76.454) (end 152.146 76.454) (width 0.508) (layer B.Cu) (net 29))
 (segment (start 147.32 74.168) (end 149.606 76.454) (width 0.508) (layer B.Cu) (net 29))
 (segment (start 144.434818 74.168) (end 147.32 74.168) (width 0.508) (layer B.Cu) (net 29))
 (segment (start 156.972 73.152) (end 157.226 73.406) (width 0.508) (layer B.Cu) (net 29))
 (segment (start 148.336 71.374) (end 151.638 74.676) (width 0.508) (layer B.Cu) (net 29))
 (segment (start 143.591409 73.324591) (end 144.434818 74.168) (width 0.508) (layer B.Cu) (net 29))
 (segment (start 153.162 73.152) (end 156.972 73.152) (width 0.508) (layer B.Cu) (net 29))
 (segment (start 150.703409 71.374) (end 151.384 71.374) (width 0.508) (layer B.Cu) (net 30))
 (segment (start 151.384 71.374) (end 153.162 73.152) (width 0.508) (layer B.Cu) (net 30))
 (segment (start 147.147409 71.374) (end 148.336 71.374) (width 0.508) (layer B.Cu) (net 31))
 (segment (start 143.591409 71.374) (end 143.591409 73.324591) (width 0.508) (layer B.Cu) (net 32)))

